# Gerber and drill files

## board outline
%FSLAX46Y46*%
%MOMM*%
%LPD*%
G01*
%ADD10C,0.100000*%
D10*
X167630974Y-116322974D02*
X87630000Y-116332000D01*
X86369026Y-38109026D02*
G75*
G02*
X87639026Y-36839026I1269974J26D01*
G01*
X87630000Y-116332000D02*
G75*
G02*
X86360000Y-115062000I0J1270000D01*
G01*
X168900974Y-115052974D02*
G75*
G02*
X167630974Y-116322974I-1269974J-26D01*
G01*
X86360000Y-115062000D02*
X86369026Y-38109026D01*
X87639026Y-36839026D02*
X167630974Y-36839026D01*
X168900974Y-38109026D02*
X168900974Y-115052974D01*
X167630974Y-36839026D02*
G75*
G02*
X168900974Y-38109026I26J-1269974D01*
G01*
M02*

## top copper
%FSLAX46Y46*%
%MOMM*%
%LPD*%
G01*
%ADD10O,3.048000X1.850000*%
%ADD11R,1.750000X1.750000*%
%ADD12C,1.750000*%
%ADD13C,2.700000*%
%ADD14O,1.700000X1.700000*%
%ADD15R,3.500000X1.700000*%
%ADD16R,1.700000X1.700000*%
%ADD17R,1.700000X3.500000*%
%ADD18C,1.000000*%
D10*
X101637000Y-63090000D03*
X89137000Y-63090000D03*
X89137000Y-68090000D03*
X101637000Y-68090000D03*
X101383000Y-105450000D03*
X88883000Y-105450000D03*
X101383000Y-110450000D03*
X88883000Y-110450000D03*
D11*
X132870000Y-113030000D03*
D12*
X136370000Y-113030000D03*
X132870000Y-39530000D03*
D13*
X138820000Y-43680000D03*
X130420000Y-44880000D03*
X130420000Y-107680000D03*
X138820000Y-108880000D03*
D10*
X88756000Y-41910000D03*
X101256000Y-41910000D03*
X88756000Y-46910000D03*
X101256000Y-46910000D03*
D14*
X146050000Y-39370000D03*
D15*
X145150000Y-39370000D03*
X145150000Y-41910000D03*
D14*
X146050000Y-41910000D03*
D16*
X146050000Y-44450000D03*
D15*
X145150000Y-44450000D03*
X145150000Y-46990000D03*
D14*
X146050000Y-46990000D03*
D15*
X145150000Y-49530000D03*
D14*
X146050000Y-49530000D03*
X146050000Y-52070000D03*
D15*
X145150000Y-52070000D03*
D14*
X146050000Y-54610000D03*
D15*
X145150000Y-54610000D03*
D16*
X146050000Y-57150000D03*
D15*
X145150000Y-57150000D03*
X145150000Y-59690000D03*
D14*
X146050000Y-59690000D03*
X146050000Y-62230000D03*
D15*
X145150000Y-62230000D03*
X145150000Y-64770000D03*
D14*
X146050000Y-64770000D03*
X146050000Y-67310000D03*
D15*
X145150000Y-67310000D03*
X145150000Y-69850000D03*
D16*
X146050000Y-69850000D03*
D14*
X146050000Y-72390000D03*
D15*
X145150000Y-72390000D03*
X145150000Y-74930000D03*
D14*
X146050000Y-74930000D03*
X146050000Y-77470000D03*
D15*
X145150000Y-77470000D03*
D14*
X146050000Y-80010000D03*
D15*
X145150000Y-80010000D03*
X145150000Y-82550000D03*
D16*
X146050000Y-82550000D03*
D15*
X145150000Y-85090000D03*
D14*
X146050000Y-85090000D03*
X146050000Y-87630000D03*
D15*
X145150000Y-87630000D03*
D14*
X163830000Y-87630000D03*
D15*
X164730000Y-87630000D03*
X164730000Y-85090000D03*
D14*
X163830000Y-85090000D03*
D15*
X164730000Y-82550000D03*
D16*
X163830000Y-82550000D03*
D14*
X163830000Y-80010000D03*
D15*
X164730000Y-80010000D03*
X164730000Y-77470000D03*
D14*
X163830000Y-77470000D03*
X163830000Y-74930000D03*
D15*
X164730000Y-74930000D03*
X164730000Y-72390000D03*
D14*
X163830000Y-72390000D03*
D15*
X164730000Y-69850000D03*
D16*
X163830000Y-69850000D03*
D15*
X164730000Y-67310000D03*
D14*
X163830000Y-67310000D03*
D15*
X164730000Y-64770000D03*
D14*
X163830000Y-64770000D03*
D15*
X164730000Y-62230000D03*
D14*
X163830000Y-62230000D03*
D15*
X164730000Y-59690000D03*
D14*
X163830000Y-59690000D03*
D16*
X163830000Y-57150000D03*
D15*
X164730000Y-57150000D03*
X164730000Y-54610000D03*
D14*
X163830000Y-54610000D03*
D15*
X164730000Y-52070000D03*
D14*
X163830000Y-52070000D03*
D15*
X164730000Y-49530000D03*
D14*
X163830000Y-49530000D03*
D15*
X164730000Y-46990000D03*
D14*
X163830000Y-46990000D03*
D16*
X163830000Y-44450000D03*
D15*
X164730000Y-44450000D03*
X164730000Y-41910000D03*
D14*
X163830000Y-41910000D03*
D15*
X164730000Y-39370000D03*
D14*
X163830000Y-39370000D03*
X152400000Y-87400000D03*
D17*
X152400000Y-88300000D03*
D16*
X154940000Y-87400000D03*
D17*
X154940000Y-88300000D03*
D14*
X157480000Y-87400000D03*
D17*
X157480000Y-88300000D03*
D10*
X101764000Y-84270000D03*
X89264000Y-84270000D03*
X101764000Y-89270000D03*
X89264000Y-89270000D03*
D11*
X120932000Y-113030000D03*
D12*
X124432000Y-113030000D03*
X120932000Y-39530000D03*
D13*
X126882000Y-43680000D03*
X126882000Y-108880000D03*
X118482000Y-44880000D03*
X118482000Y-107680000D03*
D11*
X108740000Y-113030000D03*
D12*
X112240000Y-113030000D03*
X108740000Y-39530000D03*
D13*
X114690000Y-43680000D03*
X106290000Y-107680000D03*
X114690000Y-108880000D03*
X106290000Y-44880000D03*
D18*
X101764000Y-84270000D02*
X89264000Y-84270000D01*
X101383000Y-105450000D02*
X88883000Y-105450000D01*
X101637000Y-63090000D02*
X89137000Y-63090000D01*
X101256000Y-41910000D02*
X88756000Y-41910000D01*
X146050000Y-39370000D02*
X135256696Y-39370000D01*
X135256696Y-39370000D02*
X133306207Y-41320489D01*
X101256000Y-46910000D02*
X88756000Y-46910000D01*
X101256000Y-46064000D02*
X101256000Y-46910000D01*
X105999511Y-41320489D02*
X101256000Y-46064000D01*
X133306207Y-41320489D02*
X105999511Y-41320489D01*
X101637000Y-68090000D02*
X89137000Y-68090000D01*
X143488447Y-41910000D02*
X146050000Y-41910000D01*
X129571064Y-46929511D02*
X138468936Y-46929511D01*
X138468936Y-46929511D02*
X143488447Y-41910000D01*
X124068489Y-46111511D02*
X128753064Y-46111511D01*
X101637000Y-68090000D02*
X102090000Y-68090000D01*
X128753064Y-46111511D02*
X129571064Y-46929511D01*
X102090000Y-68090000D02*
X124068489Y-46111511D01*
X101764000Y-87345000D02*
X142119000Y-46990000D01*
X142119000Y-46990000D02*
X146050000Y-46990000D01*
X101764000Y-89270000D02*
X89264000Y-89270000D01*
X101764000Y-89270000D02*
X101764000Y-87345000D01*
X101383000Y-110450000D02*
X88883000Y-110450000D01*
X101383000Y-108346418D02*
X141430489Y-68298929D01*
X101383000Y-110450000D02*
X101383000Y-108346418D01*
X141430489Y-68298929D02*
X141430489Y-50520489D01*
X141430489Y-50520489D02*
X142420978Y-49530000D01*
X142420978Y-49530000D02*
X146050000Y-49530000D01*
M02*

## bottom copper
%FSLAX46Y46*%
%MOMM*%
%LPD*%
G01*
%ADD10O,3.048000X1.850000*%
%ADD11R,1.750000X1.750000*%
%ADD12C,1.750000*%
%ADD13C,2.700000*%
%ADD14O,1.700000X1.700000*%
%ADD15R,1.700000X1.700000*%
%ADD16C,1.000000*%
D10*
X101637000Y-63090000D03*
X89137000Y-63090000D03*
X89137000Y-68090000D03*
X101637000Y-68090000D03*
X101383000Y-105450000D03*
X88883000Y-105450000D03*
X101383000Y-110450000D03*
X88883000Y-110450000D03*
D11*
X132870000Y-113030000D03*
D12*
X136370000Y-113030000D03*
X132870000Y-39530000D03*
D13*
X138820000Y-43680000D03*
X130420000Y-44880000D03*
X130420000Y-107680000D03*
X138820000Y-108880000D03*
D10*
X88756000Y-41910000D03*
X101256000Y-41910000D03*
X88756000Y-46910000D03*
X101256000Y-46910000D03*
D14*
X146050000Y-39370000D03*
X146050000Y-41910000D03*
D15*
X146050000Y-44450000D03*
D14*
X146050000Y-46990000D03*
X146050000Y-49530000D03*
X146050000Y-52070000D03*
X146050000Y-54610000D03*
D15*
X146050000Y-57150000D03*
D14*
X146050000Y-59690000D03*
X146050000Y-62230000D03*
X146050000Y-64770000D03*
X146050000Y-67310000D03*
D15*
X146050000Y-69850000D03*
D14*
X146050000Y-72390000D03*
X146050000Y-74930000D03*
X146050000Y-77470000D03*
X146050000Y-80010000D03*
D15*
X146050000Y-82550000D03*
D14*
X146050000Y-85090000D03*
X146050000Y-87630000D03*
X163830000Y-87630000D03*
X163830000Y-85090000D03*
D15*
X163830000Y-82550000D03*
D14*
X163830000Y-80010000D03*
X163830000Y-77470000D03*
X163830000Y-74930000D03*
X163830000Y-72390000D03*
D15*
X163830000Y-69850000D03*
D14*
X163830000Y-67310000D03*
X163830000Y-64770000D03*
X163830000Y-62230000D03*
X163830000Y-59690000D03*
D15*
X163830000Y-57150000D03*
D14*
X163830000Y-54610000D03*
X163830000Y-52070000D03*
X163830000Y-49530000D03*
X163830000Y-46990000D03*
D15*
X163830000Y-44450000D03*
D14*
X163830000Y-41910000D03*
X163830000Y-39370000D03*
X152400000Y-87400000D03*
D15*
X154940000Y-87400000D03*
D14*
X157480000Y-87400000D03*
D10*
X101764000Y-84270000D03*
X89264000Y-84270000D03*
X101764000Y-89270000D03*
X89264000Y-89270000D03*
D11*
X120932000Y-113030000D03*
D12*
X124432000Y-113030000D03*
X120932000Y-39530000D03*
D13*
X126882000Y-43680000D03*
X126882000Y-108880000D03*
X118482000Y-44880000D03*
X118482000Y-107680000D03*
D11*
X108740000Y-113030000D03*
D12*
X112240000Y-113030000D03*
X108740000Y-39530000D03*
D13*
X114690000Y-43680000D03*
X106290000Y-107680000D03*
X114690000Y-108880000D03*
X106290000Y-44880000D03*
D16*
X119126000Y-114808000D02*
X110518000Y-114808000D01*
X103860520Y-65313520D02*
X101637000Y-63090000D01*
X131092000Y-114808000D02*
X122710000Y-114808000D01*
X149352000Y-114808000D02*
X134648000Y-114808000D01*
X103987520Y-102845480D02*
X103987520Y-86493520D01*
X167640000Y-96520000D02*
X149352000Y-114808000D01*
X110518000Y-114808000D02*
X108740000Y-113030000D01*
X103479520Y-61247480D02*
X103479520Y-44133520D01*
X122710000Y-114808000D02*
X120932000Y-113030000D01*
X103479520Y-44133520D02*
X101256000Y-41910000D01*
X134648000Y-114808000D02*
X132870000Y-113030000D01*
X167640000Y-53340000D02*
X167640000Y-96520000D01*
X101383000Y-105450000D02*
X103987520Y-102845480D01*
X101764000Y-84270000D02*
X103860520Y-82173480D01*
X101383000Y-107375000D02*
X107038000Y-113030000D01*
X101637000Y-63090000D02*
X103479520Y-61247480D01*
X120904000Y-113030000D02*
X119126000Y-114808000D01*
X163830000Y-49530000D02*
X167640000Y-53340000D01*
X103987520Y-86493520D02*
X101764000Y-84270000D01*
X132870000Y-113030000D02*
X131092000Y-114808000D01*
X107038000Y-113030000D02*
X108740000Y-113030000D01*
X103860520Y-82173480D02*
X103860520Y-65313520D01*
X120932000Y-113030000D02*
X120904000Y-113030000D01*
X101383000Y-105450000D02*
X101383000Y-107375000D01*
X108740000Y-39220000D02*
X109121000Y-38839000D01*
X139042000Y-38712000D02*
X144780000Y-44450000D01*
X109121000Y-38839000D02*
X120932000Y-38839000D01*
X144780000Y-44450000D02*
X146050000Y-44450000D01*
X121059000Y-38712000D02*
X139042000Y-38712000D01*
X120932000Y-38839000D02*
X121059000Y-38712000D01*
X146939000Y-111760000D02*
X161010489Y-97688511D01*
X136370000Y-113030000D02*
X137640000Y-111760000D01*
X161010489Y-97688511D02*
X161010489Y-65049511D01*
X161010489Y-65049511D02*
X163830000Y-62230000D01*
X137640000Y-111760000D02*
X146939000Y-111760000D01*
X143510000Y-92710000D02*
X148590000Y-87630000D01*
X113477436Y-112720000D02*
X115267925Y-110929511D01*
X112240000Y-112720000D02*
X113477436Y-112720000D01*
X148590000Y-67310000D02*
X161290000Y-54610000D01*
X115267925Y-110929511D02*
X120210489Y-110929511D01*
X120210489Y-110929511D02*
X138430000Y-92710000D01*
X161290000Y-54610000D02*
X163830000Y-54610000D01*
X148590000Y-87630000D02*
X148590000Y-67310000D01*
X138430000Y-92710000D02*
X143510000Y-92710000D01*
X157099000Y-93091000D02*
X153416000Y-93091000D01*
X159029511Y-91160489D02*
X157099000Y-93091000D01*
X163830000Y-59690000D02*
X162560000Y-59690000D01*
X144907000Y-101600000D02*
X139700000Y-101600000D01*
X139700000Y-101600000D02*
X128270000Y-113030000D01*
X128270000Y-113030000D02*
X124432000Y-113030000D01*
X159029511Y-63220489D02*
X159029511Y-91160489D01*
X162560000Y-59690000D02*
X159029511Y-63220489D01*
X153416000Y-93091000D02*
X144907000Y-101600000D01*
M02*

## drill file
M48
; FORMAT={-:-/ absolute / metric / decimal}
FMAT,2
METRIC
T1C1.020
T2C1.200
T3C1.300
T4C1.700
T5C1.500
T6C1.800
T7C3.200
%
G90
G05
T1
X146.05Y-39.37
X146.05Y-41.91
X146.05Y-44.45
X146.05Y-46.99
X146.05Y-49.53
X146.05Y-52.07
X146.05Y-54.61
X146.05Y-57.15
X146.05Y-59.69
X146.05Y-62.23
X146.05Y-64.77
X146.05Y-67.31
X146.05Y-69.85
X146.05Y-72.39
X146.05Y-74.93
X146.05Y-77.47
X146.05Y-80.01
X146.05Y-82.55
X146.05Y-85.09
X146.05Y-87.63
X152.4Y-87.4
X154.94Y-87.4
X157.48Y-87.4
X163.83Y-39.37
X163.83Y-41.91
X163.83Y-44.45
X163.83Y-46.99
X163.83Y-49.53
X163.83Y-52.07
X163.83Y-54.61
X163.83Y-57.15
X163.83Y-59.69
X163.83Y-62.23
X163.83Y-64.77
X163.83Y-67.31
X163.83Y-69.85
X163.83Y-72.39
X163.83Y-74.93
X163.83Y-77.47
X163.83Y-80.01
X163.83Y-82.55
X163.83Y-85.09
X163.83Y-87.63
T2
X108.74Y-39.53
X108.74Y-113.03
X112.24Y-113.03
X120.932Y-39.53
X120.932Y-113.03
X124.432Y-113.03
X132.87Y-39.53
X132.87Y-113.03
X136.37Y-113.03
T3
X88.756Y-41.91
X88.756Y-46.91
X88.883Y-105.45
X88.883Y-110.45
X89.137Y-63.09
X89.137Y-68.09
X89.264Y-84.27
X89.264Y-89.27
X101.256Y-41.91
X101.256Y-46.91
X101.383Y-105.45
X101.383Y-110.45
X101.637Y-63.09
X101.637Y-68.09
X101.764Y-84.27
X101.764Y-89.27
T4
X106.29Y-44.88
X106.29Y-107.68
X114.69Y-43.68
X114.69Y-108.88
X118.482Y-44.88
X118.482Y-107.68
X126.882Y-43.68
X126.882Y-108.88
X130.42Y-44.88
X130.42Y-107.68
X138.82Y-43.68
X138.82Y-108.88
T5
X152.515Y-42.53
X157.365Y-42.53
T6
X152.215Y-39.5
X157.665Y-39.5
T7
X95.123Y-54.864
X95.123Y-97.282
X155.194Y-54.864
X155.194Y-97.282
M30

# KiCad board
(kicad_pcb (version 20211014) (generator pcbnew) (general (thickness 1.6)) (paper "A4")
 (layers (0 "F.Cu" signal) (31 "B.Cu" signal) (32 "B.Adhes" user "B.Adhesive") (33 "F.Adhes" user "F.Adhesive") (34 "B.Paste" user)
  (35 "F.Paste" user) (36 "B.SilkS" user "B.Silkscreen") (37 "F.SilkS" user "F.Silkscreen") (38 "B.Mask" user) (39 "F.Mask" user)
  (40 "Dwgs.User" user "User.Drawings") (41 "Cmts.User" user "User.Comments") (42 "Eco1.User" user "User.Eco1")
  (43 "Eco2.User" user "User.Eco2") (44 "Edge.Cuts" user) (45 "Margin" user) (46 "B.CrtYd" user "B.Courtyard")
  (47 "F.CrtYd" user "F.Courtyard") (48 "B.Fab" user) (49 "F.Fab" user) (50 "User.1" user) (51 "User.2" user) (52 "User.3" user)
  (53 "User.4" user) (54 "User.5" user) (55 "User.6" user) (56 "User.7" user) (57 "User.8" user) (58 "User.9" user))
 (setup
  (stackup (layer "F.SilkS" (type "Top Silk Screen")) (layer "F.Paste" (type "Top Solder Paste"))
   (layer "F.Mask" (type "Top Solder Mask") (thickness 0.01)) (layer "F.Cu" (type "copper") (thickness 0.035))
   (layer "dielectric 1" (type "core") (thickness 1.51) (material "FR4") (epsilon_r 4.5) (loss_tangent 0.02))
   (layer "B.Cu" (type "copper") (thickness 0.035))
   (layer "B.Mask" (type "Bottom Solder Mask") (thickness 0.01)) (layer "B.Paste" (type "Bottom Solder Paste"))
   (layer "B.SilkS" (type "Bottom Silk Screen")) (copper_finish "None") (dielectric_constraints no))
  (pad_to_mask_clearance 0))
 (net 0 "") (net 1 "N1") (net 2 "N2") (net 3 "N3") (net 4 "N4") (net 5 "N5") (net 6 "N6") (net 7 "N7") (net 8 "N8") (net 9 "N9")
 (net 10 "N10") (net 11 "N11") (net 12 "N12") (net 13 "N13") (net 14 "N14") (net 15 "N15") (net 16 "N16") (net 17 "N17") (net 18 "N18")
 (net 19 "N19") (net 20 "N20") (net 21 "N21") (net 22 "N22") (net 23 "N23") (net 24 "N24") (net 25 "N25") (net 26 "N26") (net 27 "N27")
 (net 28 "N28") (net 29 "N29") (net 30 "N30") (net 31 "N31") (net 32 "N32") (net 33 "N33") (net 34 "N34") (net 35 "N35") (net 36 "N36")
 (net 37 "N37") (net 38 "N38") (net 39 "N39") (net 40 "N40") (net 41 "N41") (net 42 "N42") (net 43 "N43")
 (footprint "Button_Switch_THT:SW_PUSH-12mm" (layer "F.Cu") (at 89.137 63.09)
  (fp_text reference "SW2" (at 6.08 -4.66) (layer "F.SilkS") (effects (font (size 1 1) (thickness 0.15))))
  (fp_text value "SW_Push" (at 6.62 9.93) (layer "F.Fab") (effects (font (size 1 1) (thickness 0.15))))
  (pad "1" thru_hole oval locked (at 12.5 0) (size 3.048 1.85) (drill 1.3) (layers *.Cu *.Mask) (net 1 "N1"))
  (pad "1" thru_hole oval locked (at 0 0) (size 3.048 1.85) (drill 1.3) (layers *.Cu *.Mask) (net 1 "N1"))
  (pad "2" thru_hole oval locked (at 0 5) (size 3.048 1.85) (drill 1.3) (layers *.Cu *.Mask) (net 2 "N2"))
  (pad "2" thru_hole oval locked (at 12.5 5) (size 3.048 1.85) (drill 1.3) (layers *.Cu *.Mask) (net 2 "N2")))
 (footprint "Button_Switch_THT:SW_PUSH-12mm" (layer "F.Cu") (at 88.883 105.45)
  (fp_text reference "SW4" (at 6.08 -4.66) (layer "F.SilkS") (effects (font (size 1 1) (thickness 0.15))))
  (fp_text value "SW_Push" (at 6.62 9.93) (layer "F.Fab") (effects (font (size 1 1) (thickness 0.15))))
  (pad "1" thru_hole oval locked (at 12.5 0) (size 3.048 1.85) (drill 1.3) (layers *.Cu *.Mask) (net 1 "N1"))
  (pad "1" thru_hole oval locked (at 0 0) (size 3.048 1.85) (drill 1.3) (layers *.Cu *.Mask) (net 1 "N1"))
  (pad "2" thru_hole oval locked (at 12.5 5) (size 3.048 1.85) (drill 1.3) (layers *.Cu *.Mask) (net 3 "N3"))
  (pad "2" thru_hole oval locked (at 0 5) (size 3.048 1.85) (drill 1.3) (layers *.Cu *.Mask) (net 3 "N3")))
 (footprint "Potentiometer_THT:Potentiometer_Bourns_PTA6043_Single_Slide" (layer "F.Cu") (at 132.87 113.03 90)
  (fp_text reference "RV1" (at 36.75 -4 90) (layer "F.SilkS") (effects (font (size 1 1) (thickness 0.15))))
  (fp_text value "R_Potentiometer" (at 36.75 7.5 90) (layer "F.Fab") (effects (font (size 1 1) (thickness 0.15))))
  (pad "1" thru_hole rect locked (at 0 0 90) (size 1.75 1.75) (drill 1.2) (layers *.Cu *.Mask) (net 1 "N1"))
  (pad "2" thru_hole circle locked (at 0 3.5 90) (size 1.75 1.75) (drill 1.2) (layers *.Cu *.Mask) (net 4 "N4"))
  (pad "3" thru_hole circle locked (at 73.5 0 90) (size 1.75 1.75) (drill 1.2) (layers *.Cu *.Mask) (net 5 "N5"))
  (pad "MP" thru_hole circle locked (at 69.35 5.95 90) (size 2.7 2.7) (drill 1.7) (layers *.Cu *.Mask))
  (pad "MP" thru_hole circle locked (at 68.15 -2.45 90) (size 2.7 2.7) (drill 1.7) (layers *.Cu *.Mask))
  (pad "MP" thru_hole circle locked (at 5.35 -2.45 90) (size 2.7 2.7) (drill 1.7) (layers *.Cu *.Mask))
  (pad "MP" thru_hole circle locked (at 4.15 5.95 90) (size 2.7 2.7) (drill 1.7) (layers *.Cu *.Mask)))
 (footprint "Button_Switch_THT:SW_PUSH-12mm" (layer "F.Cu") (at 88.756 41.91)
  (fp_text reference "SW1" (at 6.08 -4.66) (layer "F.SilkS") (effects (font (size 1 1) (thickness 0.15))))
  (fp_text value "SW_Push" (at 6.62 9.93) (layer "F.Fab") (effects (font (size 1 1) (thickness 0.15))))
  (pad "1" thru_hole oval locked (at 0 0) (size 3.048 1.85) (drill 1.3) (layers *.Cu *.Mask) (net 1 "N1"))
  (pad "1" thru_hole oval locked (at 12.5 0) (size 3.048 1.85) (drill 1.3) (layers *.Cu *.Mask) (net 1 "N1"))
  (pad "2" thru_hole oval locked (at 0 5) (size 3.048 1.85) (drill 1.3) (layers *.Cu *.Mask) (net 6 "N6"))
  (pad "2" thru_hole oval locked (at 12.5 5) (size 3.048 1.85) (drill 1.3) (layers *.Cu *.Mask) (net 6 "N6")))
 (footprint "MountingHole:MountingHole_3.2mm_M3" (layer "F.Cu") (at 155.194 97.282)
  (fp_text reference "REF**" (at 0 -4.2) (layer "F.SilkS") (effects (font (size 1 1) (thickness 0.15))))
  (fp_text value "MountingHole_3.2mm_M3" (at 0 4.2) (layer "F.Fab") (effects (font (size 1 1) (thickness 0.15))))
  (pad "" np_thru_hole circle locked (at 0 0) (size 3.2 3.2) (drill 3.2) (layers *.Cu *.Mask)))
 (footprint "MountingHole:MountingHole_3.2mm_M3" (layer "F.Cu") (at 155.194 54.864)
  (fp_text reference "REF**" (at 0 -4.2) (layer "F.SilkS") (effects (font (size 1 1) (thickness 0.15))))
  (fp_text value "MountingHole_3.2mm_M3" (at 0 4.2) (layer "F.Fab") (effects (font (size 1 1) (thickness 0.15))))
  (pad "" np_thru_hole circle locked (at 0 0) (size 3.2 3.2) (drill 3.2) (layers *.Cu *.Mask)))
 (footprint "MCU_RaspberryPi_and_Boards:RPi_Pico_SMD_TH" (layer "F.Cu") (at 154.94 63.5)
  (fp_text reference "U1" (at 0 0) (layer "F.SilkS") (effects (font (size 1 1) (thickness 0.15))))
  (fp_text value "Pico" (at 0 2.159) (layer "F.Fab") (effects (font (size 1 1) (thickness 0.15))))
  (pad "" np_thru_hole oval (at -2.725 -24) (size 1.8 1.8) (drill 1.8) (layers *.Cu *.Mask))
  (pad "" np_thru_hole oval (at -2.425 -20.97) (size 1.5 1.5) (drill 1.5) (layers *.Cu *.Mask))
  (pad "" np_thru_hole oval (at 2.725 -24) (size 1.8 1.8) (drill 1.8) (layers *.Cu *.Mask))
  (pad "" np_thru_hole oval (at 2.425 -20.97) (size 1.5 1.5) (drill 1.5) (layers *.Cu *.Mask))
  (pad "1" thru_hole oval (at -8.89 -24.13) (size 1.7 1.7) (drill 1.02) (layers *.Cu *.Mask) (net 6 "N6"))
  (pad "1" smd rect (at -8.89 -24.13) (size 3.5 1.7) (drill (offset -0.9 0)) (layers "F.Cu" "F.Mask") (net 6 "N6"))
  (pad "2" smd rect (at -8.89 -21.59) (size 3.5 1.7) (drill (offset -0.9 0)) (layers "F.Cu" "F.Mask") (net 2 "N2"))
  (pad "2" thru_hole oval (at -8.89 -21.59) (size 1.7 1.7) (drill 1.02) (layers *.Cu *.Mask) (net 2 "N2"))
  (pad "3" thru_hole rect (at -8.89 -19.05) (size 1.7 1.7) (drill 1.02) (layers *.Cu *.Mask) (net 5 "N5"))
  (pad "3" smd rect (at -8.89 -19.05) (size 3.5 1.7) (drill (offset -0.9 0)) (layers "F.Cu" "F.Mask") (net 5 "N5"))
  (pad "4" smd rect (at -8.89 -16.51) (size 3.5 1.7) (drill (offset -0.9 0)) (layers "F.Cu" "F.Mask") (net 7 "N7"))
  (pad "4" thru_hole oval (at -8.89 -16.51) (size 1.7 1.7) (drill 1.02) (layers *.Cu *.Mask) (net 7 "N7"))
  (pad "5" smd rect (at -8.89 -13.97) (size 3.5 1.7) (drill (offset -0.9 0)) (layers "F.Cu" "F.Mask") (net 3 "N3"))
  (pad "5" thru_hole oval (at -8.89 -13.97) (size 1.7 1.7) (drill 1.02) (layers *.Cu *.Mask) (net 3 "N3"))
  (pad "6" thru_hole oval (at -8.89 -11.43) (size 1.7 1.7) (drill 1.02) (layers *.Cu *.Mask) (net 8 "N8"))
  (pad "6" smd rect (at -8.89 -11.43) (size 3.5 1.7) (drill (offset -0.9 0)) (layers "F.Cu" "F.Mask") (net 8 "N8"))
  (pad "7" thru_hole oval (at -8.89 -8.89) (size 1.7 1.7) (drill 1.02) (layers *.Cu *.Mask) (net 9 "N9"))
  (pad "7" smd rect (at -8.89 -8.89) (size 3.5 1.7) (drill (offset -0.9 0)) (layers "F.Cu" "F.Mask") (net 9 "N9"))
  (pad "8" thru_hole rect (at -8.89 -6.35) (size 1.7 1.7) (drill 1.02) (layers *.Cu *.Mask) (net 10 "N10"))
  (pad "8" smd rect (at -8.89 -6.35) (size 3.5 1.7) (drill (offset -0.9 0)) (layers "F.Cu" "F.Mask") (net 10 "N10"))
  (pad "9" smd rect (at -8.89 -3.81) (size 3.5 1.7) (drill (offset -0.9 0)) (layers "F.Cu" "F.Mask") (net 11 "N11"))
  (pad "9" thru_hole oval (at -8.89 -3.81) (size 1.7 1.7) (drill 1.02) (layers *.Cu *.Mask) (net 11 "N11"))
  (pad "10" thru_hole oval (at -8.89 -1.27) (size 1.7 1.7) (drill 1.02) (layers *.Cu *.Mask) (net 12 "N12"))
  (pad "10" smd rect (at -8.89 -1.27) (size 3.5 1.7) (drill (offset -0.9 0)) (layers "F.Cu" "F.Mask") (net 12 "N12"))
  (pad "11" smd rect (at -8.89 1.27) (size 3.5 1.7) (drill (offset -0.9 0)) (layers "F.Cu" "F.Mask") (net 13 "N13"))
  (pad "11" thru_hole oval (at -8.89 1.27) (size 1.7 1.7) (drill 1.02) (layers *.Cu *.Mask) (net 13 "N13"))
  (pad "12" thru_hole oval (at -8.89 3.81) (size 1.7 1.7) (drill 1.02) (layers *.Cu *.Mask) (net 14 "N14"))
  (pad "12" smd rect (at -8.89 3.81) (size 3.5 1.7) (drill (offset -0.9 0)) (layers "F.Cu" "F.Mask") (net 14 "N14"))
  (pad "13" smd rect (at -8.89 6.35) (size 3.5 1.7) (drill (offset -0.9 0)) (layers "F.Cu" "F.Mask") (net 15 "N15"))
  (pad "13" thru_hole rect (at -8.89 6.35) (size 1.7 1.7) (drill 1.02) (layers *.Cu *.Mask) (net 15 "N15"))
  (pad "14" thru_hole oval (at -8.89 8.89) (size 1.7 1.7) (drill 1.02) (layers *.Cu *.Mask) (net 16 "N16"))
  (pad "14" smd rect (at -8.89 8.89) (size 3.5 1.7) (drill (offset -0.9 0)) (layers "F.Cu" "F.Mask") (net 16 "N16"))
  (pad "15" smd rect (at -8.89 11.43) (size 3.5 1.7) (drill (offset -0.9 0)) (layers "F.Cu" "F.Mask") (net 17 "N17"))
  (pad "15" thru_hole oval (at -8.89 11.43) (size 1.7 1.7) (drill 1.02) (layers *.Cu *.Mask) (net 17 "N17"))
  (pad "16" thru_hole oval (at -8.89 13.97) (size 1.7 1.7) (drill 1.02) (layers *.Cu *.Mask) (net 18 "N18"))
  (pad "16" smd rect (at -8.89 13.97) (size 3.5 1.7) (drill (offset -0.9 0)) (layers "F.Cu" "F.Mask") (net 18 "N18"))
  (pad "17" thru_hole oval (at -8.89 16.51) (size 1.7 1.7) (drill 1.02) (layers *.Cu *.Mask) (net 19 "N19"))
  (pad "17" smd rect (at -8.89 16.51) (size 3.5 1.7) (drill (offset -0.9 0)) (layers "F.Cu" "F.Mask") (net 19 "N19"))
  (pad "18" smd rect (at -8.89 19.05) (size 3.5 1.7) (drill (offset -0.9 0)) (layers "F.Cu" "F.Mask") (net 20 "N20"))
  (pad "18" thru_hole rect (at -8.89 19.05) (size 1.7 1.7) (drill 1.02) (layers *.Cu *.Mask) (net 20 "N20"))
  (pad "19" smd rect (at -8.89 21.59) (size 3.5 1.7) (drill (offset -0.9 0)) (layers "F.Cu" "F.Mask") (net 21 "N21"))
  (pad "19" thru_hole oval (at -8.89 21.59) (size 1.7 1.7) (drill 1.02) (layers *.Cu *.Mask) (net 21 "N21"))
  (pad "20" thru_hole oval (at -8.89 24.13) (size 1.7 1.7) (drill 1.02) (layers *.Cu *.Mask) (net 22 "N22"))
  (pad "20" smd rect (at -8.89 24.13) (size 3.5 1.7) (drill (offset -0.9 0)) (layers "F.Cu" "F.Mask") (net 22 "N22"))
  (pad "21" thru_hole oval (at 8.89 24.13) (size 1.7 1.7) (drill 1.02) (layers *.Cu *.Mask) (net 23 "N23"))
  (pad "21" smd rect (at 8.89 24.13) (size 3.5 1.7) (drill (offset 0.9 0)) (layers "F.Cu" "F.Mask") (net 23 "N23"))
  (pad "22" smd rect (at 8.89 21.59) (size 3.5 1.7) (drill (offset 0.9 0)) (layers "F.Cu" "F.Mask") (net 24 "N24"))
  (pad "22" thru_hole oval (at 8.89 21.59) (size 1.7 1.7) (drill 1.02) (layers *.Cu *.Mask) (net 24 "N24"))
  (pad "23" smd rect (at 8.89 19.05) (size 3.5 1.7) (drill (offset 0.9 0)) (layers "F.Cu" "F.Mask") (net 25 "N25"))
  (pad "23" thru_hole rect (at 8.89 19.05) (size 1.7 1.7) (drill 1.02) (layers *.Cu *.Mask) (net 25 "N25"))
  (pad "24" thru_hole oval (at 8.89 16.51) (size 1.7 1.7) (drill 1.02) (layers *.Cu *.Mask) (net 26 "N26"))
  (pad "24" smd rect (at 8.89 16.51) (size 3.5 1.7) (drill (offset 0.9 0)) (layers "F.Cu" "F.Mask") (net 26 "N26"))
  (pad "25" smd rect (at 8.89 13.97) (size 3.5 1.7) (drill (offset 0.9 0)) (layers "F.Cu" "F.Mask") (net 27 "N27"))
  (pad "25" thru_hole oval (at 8.89 13.97) (size 1.7 1.7) (drill 1.02) (layers *.Cu *.Mask) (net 27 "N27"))
  (pad "26" thru_hole oval (at 8.89 11.43) (size 1.7 1.7) (drill 1.02) (layers *.Cu *.Mask) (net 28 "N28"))
  (pad "26" smd rect (at 8.89 11.43) (size 3.5 1.7) (drill (offset 0.9 0)) (layers "F.Cu" "F.Mask") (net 28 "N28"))
  (pad "27" smd rect (at 8.89 8.89) (size 3.5 1.7) (drill (offset 0.9 0)) (layers "F.Cu" "F.Mask") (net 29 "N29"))
  (pad "27" thru_hole oval (at 8.89 8.89) (size 1.7 1.7) (drill 1.02) (layers *.Cu *.Mask) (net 29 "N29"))
  (pad "28" smd rect (at 8.89 6.35) (size 3.5 1.7) (drill (offset 0.9 0)) (layers "F.Cu" "F.Mask") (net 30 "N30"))
  (pad "28" thru_hole rect (at 8.89 6.35) (size 1.7 1.7) (drill 1.02) (layers *.Cu *.Mask) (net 30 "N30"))
  (pad "29" smd rect (at 8.89 3.81) (size 3.5 1.7) (drill (offset 0.9 0)) (layers "F.Cu" "F.Mask") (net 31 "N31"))
  (pad "29" thru_hole oval (at 8.89 3.81) (size 1.7 1.7) (drill 1.02) (layers *.Cu *.Mask) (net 31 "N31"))
  (pad "30" smd rect (at 8.89 1.27) (size 3.5 1.7) (drill (offset 0.9 0)) (layers "F.Cu" "F.Mask") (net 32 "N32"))
  (pad "30" thru_hole oval (at 8.89 1.27) (size 1.7 1.7) (drill 1.02) (layers *.Cu *.Mask) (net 32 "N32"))
  (pad "31" smd rect (at 8.89 -1.27) (size 3.5 1.7) (drill (offset 0.9 0)) (layers "F.Cu" "F.Mask") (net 4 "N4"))
  (pad "31" thru_hole oval (at 8.89 -1.27) (size 1.7 1.7) (drill 1.02) (layers *.Cu *.Mask) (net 4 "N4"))
  (pad "32" smd rect (at 8.89 -3.81) (size 3.5 1.7) (drill (offset 0.9 0)) (layers "F.Cu" "F.Mask") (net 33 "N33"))
  (pad "32" thru_hole oval (at 8.89 -3.81) (size 1.7 1.7) (drill 1.02) (layers *.Cu *.Mask) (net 33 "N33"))
  (pad "33" thru_hole rect (at 8.89 -6.35) (size 1.7 1.7) (drill 1.02) (layers *.Cu *.Mask) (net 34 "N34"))
  (pad "33" smd rect (at 8.89 -6.35) (size 3.5 1.7) (drill (offset 0.9 0)) (layers "F.Cu" "F.Mask") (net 34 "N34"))
  (pad "34" smd rect (at 8.89 -8.89) (size 3.5 1.7) (drill (offset 0.9 0)) (layers "F.Cu" "F.Mask") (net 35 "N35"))
  (pad "34" thru_hole oval (at 8.89 -8.89) (size 1.7 1.7) (drill 1.02) (layers *.Cu *.Mask) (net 35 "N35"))
  (pad "35" smd rect (at 8.89 -11.43) (size 3.5 1.7) (drill (offset 0.9 0)) (layers "F.Cu" "F.Mask") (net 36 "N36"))
  (pad "35" thru_hole oval (at 8.89 -11.43) (size 1.7 1.7) (drill 1.02) (layers *.Cu *.Mask) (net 36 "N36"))
  (pad "36" smd rect (at 8.89 -13.97) (size 3.5 1.7) (drill (offset 0.9 0)) (layers "F.Cu" "F.Mask") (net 1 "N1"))
  (pad "36" thru_hole oval (at 8.89 -13.97) (size 1.7 1.7) (drill 1.02) (layers *.Cu *.Mask) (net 1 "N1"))
  (pad "37" smd rect (at 8.89 -16.51) (size 3.5 1.7) (drill (offset 0.9 0)) (layers "F.Cu" "F.Mask") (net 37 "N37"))
  (pad "37" thru_hole oval (at 8.89 -16.51) (size 1.7 1.7) (drill 1.02) (layers *.Cu *.Mask) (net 37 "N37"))
  (pad "38" thru_hole rect (at 8.89 -19.05) (size 1.7 1.7) (drill 1.02) (layers *.Cu *.Mask) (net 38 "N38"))
  (pad "38" smd rect (at 8.89 -19.05) (size 3.5 1.7) (drill (offset 0.9 0)) (layers "F.Cu" "F.Mask") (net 38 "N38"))
  (pad "39" smd rect (at 8.89 -21.59) (size 3.5 1.7) (drill (offset 0.9 0)) (layers "F.Cu" "F.Mask") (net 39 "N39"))
  (pad "39" thru_hole oval (at 8.89 -21.59) (size 1.7 1.7) (drill 1.02) (layers *.Cu *.Mask) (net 39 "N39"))
  (pad "40" smd rect (at 8.89 -24.13) (size 3.5 1.7) (drill (offset 0.9 0)) (layers "F.Cu" "F.Mask") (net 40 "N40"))
  (pad "40" thru_hole oval (at 8.89 -24.13) (size 1.7 1.7) (drill 1.02) (layers *.Cu *.Mask) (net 40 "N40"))
  (pad "41" thru_hole oval (at -2.54 23.9) (size 1.7 1.7) (drill 1.02) (layers *.Cu *.Mask) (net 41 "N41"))
  (pad "41" smd rect (at -2.54 23.9 90) (size 3.5 1.7) (drill (offset -0.9 0)) (layers "F.Cu" "F.Mask") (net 41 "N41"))
  (pad "42" thru_hole rect (at 0 23.9) (size 1.7 1.7) (drill 1.02) (layers *.Cu *.Mask) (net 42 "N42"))
  (pad "42" smd rect (at 0 23.9 90) (size 3.5 1.7) (drill (offset -0.9 0)) (layers "F.Cu" "F.Mask") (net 42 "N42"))
  (pad "43" thru_hole oval (at 2.54 23.9) (size 1.7 1.7) (drill 1.02) (layers *.Cu *.Mask) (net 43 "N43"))
  (pad "43" smd rect (at 2.54 23.9 90) (size 3.5 1.7) (drill (offset -0.9 0)) (layers "F.Cu" "F.Mask") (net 43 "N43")))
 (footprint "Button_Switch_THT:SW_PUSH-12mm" (layer "F.Cu") (at 89.264 84.27)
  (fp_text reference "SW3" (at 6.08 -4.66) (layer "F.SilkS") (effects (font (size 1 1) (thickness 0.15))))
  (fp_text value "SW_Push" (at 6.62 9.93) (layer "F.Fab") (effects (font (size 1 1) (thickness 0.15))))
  (pad "1" thru_hole oval locked (at 12.5 0) (size 3.048 1.85) (drill 1.3) (layers *.Cu *.Mask) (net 1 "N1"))
  (pad "1" thru_hole oval locked (at 0 0) (size 3.048 1.85) (drill 1.3) (layers *.Cu *.Mask) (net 1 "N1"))
  (pad "2" thru_hole oval locked (at 12.5 5) (size 3.048 1.85) (drill 1.3) (layers *.Cu *.Mask) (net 7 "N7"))
  (pad "2" thru_hole oval locked (at 0 5) (size 3.048 1.85) (drill 1.3) (layers *.Cu *.Mask) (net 7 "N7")))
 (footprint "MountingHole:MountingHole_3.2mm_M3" (layer "F.Cu") (at 95.123 54.864)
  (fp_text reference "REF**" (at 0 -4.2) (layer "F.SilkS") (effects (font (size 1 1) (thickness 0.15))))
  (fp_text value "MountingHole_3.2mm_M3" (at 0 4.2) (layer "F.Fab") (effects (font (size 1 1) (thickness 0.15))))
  (pad "" np_thru_hole circle locked (at 0 0) (size 3.2 3.2) (drill 3.2) (layers *.Cu *.Mask)))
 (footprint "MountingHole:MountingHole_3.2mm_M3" (layer "F.Cu") (at 95.123 97.282)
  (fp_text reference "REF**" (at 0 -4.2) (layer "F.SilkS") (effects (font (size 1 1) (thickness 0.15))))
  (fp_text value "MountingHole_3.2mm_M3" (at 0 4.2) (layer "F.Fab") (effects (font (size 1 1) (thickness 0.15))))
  (pad "" np_thru_hole circle locked (at 0 0) (size 3.2 3.2) (drill 3.2) (layers *.Cu *.Mask)))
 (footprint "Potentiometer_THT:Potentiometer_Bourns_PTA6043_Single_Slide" (layer "F.Cu") (at 120.932 113.03 90)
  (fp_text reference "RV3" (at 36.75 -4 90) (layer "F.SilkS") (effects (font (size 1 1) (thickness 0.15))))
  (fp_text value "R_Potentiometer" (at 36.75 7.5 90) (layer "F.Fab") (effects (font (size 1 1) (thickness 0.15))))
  (pad "1" thru_hole rect locked (at 0 0 90) (size 1.75 1.75) (drill 1.2) (layers *.Cu *.Mask) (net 1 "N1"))
  (pad "2" thru_hole circle locked (at 0 3.5 90) (size 1.75 1.75) (drill 1.2) (layers *.Cu *.Mask) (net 33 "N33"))
  (pad "3" thru_hole circle locked (at 73.5 0 90) (size 1.75 1.75) (drill 1.2) (layers *.Cu *.Mask) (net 5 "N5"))
  (pad "MP" thru_hole circle locked (at 69.35 5.95 90) (size 2.7 2.7) (drill 1.7) (layers *.Cu *.Mask))
  (pad "MP" thru_hole circle locked (at 4.15 5.95 90) (size 2.7 2.7) (drill 1.7) (layers *.Cu *.Mask))
  (pad "MP" thru_hole circle locked (at 68.15 -2.45 90) (size 2.7 2.7) (drill 1.7) (layers *.Cu *.Mask))
  (pad "MP" thru_hole circle locked (at 5.35 -2.45 90) (size 2.7 2.7) (drill 1.7) (layers *.Cu *.Mask)))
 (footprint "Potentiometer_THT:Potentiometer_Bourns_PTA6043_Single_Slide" (layer "F.Cu") (at 108.74 113.03 90)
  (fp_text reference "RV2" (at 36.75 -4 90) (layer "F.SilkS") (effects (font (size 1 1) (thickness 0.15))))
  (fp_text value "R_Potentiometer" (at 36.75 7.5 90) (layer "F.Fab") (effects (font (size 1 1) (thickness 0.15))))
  (pad "1" thru_hole rect locked (at 0 0 90) (size 1.75 1.75) (drill 1.2) (layers *.Cu *.Mask) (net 1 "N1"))
  (pad "2" thru_hole circle locked (at 0 3.5 90) (size 1.75 1.75) (drill 1.2) (layers *.Cu *.Mask) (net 35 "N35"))
  (pad "3" thru_hole circle locked (at 73.5 0 90) (size 1.75 1.75) (drill 1.2) (layers *.Cu *.Mask) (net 5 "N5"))
  (pad "MP" thru_hole circle locked (at 69.35 5.95 90) (size 2.7 2.7) (drill 1.7) (layers *.Cu *.Mask))
  (pad "MP" thru_hole circle locked (at 5.35 -2.45 90) (size 2.7 2.7) (drill 1.7) (layers *.Cu *.Mask))
  (pad "MP" thru_hole circle locked (at 4.15 5.95 90) (size 2.7 2.7) (drill 1.7) (layers *.Cu *.Mask))
  (pad "MP" thru_hole circle locked (at 68.15 -2.45 90) (size 2.7 2.7) (drill 1.7) (layers *.Cu *.Mask)))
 (gr_line (start 167.630974 116.322974) (end 87.63 116.332) (layer "Edge.Cuts") (width 0.1))
 (gr_arc (start 86.369026 38.109026) (mid 86.741 37.211) (end 87.639026 36.839026) (layer "Edge.Cuts") (width 0.1))
 (gr_arc (start 87.63 116.332) (mid 86.731974 115.960026) (end 86.36 115.062) (layer "Edge.Cuts") (width 0.1))
 (gr_arc (start 168.900974 115.052974) (mid 168.529 115.951) (end 167.630974 116.322974) (layer "Edge.Cuts") (width 0.1))
 (gr_line (start 86.36 115.062) (end 86.369026 38.109026) (layer "Edge.Cuts") (width 0.1))
 (gr_line (start 87.639026 36.839026) (end 167.630974 36.839026) (layer "Edge.Cuts") (width 0.1))
 (gr_line (start 168.900974 38.109026) (end 168.900974 115.052974) (layer "Edge.Cuts") (width 0.1))
 (gr_arc (start 167.630974 36.839026) (mid 168.529 37.211) (end 168.900974 38.109026) (layer "Edge.Cuts") (width 0.1))
 (segment (start 101.764 84.27) (end 89.264 84.27) (width 1) (layer "F.Cu") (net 1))
 (segment (start 101.383 105.45) (end 88.883 105.45) (width 1) (layer "F.Cu") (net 1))
 (segment (start 101.637 63.09) (end 89.137 63.09) (width 1) (layer "F.Cu") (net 1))
 (segment (start 101.256 41.91) (end 88.756 41.91) (width 1) (layer "F.Cu") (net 1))
 (segment (start 119.126 114.808) (end 110.518 114.808) (width 1) (layer "B.Cu") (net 1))
 (segment (start 103.86052 65.31352) (end 101.637 63.09) (width 1) (layer "B.Cu") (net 1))
 (segment (start 131.092 114.808) (end 122.71 114.808) (width 1) (layer "B.Cu") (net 1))
 (segment (start 149.352 114.808) (end 134.648 114.808) (width 1) (layer "B.Cu") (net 1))
 (segment (start 103.98752 102.84548) (end 103.98752 86.49352) (width 1) (layer "B.Cu") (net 1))
 (segment (start 167.64 96.52) (end 149.352 114.808) (width 1) (layer "B.Cu") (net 1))
 (segment (start 110.518 114.808) (end 108.74 113.03) (width 1) (layer "B.Cu") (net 1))
 (segment (start 103.47952 61.24748) (end 103.47952 44.13352) (width 1) (layer "B.Cu") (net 1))
 (segment (start 122.71 114.808) (end 120.932 113.03) (width 1) (layer "B.Cu") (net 1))
 (segment (start 103.47952 44.13352) (end 101.256 41.91) (width 1) (layer "B.Cu") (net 1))
 (segment (start 134.648 114.808) (end 132.87 113.03) (width 1) (layer "B.Cu") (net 1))
 (segment (start 167.64 53.34) (end 167.64 96.52) (width 1) (layer "B.Cu") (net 1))
 (segment (start 101.383 105.45) (end 103.98752 102.84548) (width 1) (layer "B.Cu") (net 1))
 (segment (start 101.764 84.27) (end 103.86052 82.17348) (width 1) (layer "B.Cu") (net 1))
 (segment (start 101.383 107.375) (end 107.038 113.03) (width 1) (layer "B.Cu") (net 1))
 (segment (start 101.637 63.09) (end 103.47952 61.24748) (width 1) (layer "B.Cu") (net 1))
 (segment (start 120.904 113.03) (end 119.126 114.808) (width 1) (layer "B.Cu") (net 1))
 (segment (start 163.83 49.53) (end 167.64 53.34) (width 1) (layer "B.Cu") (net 1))
 (segment (start 103.98752 86.49352) (end 101.764 84.27) (width 1) (layer "B.Cu") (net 1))
 (segment (start 132.87 113.03) (end 131.092 114.808) (width 1) (layer "B.Cu") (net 1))
 (segment (start 107.038 113.03) (end 108.74 113.03) (width 1) (layer "B.Cu") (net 1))
 (segment (start 103.86052 82.17348) (end 103.86052 65.31352) (width 1) (layer "B.Cu") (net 1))
 (segment (start 120.932 113.03) (end 120.904 113.03) (width 1) (layer "B.Cu") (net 1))
 (segment (start 101.383 105.45) (end 101.383 107.375) (width 1) (layer "B.Cu") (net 1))
 (segment (start 108.74 39.22) (end 109.121 38.839) (width 1) (layer "B.Cu") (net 5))
 (segment (start 139.042 38.712) (end 144.78 44.45) (width 1) (layer "B.Cu") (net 5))
 (segment (start 109.121 38.839) (end 120.932 38.839) (width 1) (layer "B.Cu") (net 5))
 (segment (start 144.78 44.45) (end 146.05 44.45) (width 1) (layer "B.Cu") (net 5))
 (segment (start 121.059 38.712) (end 139.042 38.712) (width 1) (layer "B.Cu") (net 5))
 (segment (start 120.932 38.839) (end 121.059 38.712) (width 1) (layer "B.Cu") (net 5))
 (segment (start 146.05 39.37) (end 135.256696 39.37) (width 1) (layer "F.Cu") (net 6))
 (segment (start 135.256696 39.37) (end 133.306207 41.320489) (width 1) (layer "F.Cu") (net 6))
 (segment (start 101.256 46.91) (end 88.756 46.91) (width 1) (layer "F.Cu") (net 6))
 (segment (start 101.256 46.064) (end 101.256 46.91) (width 1) (layer "F.Cu") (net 6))
 (segment (start 105.999511 41.320489) (end 101.256 46.064) (width 1) (layer "F.Cu") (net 6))
 (segment (start 133.306207 41.320489) (end 105.999511 41.320489) (width 1) (layer "F.Cu") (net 6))
 (segment (start 101.637 68.09) (end 89.137 68.09) (width 1) (layer "F.Cu") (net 2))
 (segment (start 143.488447 41.91) (end 146.05 41.91) (width 1) (layer "F.Cu") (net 2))
 (segment (start 129.571064 46.929511) (end 138.468936 46.929511) (width 1) (layer "F.Cu") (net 2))
 (segment (start 138.468936 46.929511) (end 143.488447 41.91) (width 1) (layer "F.Cu") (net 2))
 (segment (start 124.068489 46.111511) (end 128.753064 46.111511) (width 1) (layer "F.Cu") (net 2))
 (segment (start 101.637 68.09) (end 102.09 68.09) (width 1) (layer "F.Cu") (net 2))
 (segment (start 128.753064 46.111511) (end 129.571064 46.929511) (width 1) (layer "F.Cu") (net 2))
 (segment (start 102.09 68.09) (end 124.068489 46.111511) (width 1) (layer "F.Cu") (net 2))
 (segment (start 101.764 87.345) (end 142.119 46.99) (width 1) (layer "F.Cu") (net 7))
 (segment (start 142.119 46.99) (end 146.05 46.99) (width 1) (layer "F.Cu") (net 7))
 (segment (start 101.764 89.27) (end 89.264 89.27) (width 1) (layer "F.Cu") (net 7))
 (segment (start 101.764 89.27) (end 101.764 87.345) (width 1) (layer "F.Cu") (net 7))
 (segment (start 101.383 110.45) (end 88.883 110.45) (width 1) (layer "F.Cu") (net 3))
 (segment (start 101.383 108.346418) (end 141.430489 68.298929) (width 1) (layer "F.Cu") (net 3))
 (segment (start 101.383 110.45) (end 101.383 108.346418) (width 1) (layer "F.Cu") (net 3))
 (segment (start 141.430489 68.298929) (end 141.430489 50.520489) (width 1) (layer "F.Cu") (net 3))
 (segment (start 141.430489 50.520489) (end 142.420978 49.53) (width 1) (layer "F.Cu") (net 3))
 (segment (start 142.420978 49.53) (end 146.05 49.53) (width 1) (layer "F.Cu") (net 3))
 (segment (start 146.939 111.76) (end 161.010489 97.688511) (width 1) (layer "B.Cu") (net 4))
 (segment (start 136.37 113.03) (end 137.64 111.76) (width 1) (layer "B.Cu") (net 4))
 (segment (start 161.010489 97.688511) (end 161.010489 65.049511) (width 1) (layer "B.Cu") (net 4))
 (segment (start 161.010489 65.049511) (end 163.83 62.23) (width 1) (layer "B.Cu") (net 4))
 (segment (start 137.64 111.76) (end 146.939 111.76) (width 1) (layer "B.Cu") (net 4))
 (segment (start 143.51 92.71) (end 148.59 87.63) (width 1) (layer "B.Cu") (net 35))
 (segment (start 113.477436 112.72) (end 115.267925 110.929511) (width 1) (layer "B.Cu") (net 35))
 (segment (start 112.24 112.72) (end 113.477436 112.72) (width 1) (layer "B.Cu") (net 35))
 (segment (start 148.59 67.31) (end 161.29 54.61) (width 1) (layer "B.Cu") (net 35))
 (segment (start 115.267925 110.929511) (end 120.210489 110.929511) (width 1) (layer "B.Cu") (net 35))
 (segment (start 120.210489 110.929511) (end 138.43 92.71) (width 1) (layer "B.Cu") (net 35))
 (segment (start 161.29 54.61) (end 163.83 54.61) (width 1) (layer "B.Cu") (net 35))
 (segment (start 148.59 87.63) (end 148.59 67.31) (width 1) (layer "B.Cu") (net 35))
 (segment (start 138.43 92.71) (end 143.51 92.71) (width 1) (layer "B.Cu") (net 35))
 (segment (start 157.099 93.091) (end 153.416 93.091) (width 1) (layer "B.Cu") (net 33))
 (segment (start 159.029511 91.160489) (end 157.099 93.091) (width 1) (layer "B.Cu") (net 33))
 (segment (start 163.83 59.69) (end 162.56 59.69) (width 1) (layer "B.Cu") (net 33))
 (segment (start 144.907 101.6) (end 139.7 101.6) (width 1) (layer "B.Cu") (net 33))
 (segment (start 139.7 101.6) (end 128.27 113.03) (width 1) (layer "B.Cu") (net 33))
 (segment (start 128.27 113.03) (end 124.432 113.03) (width 1) (layer "B.Cu") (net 33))
 (segment (start 159.029511 63.220489) (end 159.029511 91.160489) (width 1) (layer "B.Cu") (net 33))
 (segment (start 162.56 59.69) (end 159.029511 63.220489) (width 1) (layer "B.Cu") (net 33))
 (segment (start 153.416 93.091) (end 144.907 101.6) (width 1) (layer "B.Cu") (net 33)))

